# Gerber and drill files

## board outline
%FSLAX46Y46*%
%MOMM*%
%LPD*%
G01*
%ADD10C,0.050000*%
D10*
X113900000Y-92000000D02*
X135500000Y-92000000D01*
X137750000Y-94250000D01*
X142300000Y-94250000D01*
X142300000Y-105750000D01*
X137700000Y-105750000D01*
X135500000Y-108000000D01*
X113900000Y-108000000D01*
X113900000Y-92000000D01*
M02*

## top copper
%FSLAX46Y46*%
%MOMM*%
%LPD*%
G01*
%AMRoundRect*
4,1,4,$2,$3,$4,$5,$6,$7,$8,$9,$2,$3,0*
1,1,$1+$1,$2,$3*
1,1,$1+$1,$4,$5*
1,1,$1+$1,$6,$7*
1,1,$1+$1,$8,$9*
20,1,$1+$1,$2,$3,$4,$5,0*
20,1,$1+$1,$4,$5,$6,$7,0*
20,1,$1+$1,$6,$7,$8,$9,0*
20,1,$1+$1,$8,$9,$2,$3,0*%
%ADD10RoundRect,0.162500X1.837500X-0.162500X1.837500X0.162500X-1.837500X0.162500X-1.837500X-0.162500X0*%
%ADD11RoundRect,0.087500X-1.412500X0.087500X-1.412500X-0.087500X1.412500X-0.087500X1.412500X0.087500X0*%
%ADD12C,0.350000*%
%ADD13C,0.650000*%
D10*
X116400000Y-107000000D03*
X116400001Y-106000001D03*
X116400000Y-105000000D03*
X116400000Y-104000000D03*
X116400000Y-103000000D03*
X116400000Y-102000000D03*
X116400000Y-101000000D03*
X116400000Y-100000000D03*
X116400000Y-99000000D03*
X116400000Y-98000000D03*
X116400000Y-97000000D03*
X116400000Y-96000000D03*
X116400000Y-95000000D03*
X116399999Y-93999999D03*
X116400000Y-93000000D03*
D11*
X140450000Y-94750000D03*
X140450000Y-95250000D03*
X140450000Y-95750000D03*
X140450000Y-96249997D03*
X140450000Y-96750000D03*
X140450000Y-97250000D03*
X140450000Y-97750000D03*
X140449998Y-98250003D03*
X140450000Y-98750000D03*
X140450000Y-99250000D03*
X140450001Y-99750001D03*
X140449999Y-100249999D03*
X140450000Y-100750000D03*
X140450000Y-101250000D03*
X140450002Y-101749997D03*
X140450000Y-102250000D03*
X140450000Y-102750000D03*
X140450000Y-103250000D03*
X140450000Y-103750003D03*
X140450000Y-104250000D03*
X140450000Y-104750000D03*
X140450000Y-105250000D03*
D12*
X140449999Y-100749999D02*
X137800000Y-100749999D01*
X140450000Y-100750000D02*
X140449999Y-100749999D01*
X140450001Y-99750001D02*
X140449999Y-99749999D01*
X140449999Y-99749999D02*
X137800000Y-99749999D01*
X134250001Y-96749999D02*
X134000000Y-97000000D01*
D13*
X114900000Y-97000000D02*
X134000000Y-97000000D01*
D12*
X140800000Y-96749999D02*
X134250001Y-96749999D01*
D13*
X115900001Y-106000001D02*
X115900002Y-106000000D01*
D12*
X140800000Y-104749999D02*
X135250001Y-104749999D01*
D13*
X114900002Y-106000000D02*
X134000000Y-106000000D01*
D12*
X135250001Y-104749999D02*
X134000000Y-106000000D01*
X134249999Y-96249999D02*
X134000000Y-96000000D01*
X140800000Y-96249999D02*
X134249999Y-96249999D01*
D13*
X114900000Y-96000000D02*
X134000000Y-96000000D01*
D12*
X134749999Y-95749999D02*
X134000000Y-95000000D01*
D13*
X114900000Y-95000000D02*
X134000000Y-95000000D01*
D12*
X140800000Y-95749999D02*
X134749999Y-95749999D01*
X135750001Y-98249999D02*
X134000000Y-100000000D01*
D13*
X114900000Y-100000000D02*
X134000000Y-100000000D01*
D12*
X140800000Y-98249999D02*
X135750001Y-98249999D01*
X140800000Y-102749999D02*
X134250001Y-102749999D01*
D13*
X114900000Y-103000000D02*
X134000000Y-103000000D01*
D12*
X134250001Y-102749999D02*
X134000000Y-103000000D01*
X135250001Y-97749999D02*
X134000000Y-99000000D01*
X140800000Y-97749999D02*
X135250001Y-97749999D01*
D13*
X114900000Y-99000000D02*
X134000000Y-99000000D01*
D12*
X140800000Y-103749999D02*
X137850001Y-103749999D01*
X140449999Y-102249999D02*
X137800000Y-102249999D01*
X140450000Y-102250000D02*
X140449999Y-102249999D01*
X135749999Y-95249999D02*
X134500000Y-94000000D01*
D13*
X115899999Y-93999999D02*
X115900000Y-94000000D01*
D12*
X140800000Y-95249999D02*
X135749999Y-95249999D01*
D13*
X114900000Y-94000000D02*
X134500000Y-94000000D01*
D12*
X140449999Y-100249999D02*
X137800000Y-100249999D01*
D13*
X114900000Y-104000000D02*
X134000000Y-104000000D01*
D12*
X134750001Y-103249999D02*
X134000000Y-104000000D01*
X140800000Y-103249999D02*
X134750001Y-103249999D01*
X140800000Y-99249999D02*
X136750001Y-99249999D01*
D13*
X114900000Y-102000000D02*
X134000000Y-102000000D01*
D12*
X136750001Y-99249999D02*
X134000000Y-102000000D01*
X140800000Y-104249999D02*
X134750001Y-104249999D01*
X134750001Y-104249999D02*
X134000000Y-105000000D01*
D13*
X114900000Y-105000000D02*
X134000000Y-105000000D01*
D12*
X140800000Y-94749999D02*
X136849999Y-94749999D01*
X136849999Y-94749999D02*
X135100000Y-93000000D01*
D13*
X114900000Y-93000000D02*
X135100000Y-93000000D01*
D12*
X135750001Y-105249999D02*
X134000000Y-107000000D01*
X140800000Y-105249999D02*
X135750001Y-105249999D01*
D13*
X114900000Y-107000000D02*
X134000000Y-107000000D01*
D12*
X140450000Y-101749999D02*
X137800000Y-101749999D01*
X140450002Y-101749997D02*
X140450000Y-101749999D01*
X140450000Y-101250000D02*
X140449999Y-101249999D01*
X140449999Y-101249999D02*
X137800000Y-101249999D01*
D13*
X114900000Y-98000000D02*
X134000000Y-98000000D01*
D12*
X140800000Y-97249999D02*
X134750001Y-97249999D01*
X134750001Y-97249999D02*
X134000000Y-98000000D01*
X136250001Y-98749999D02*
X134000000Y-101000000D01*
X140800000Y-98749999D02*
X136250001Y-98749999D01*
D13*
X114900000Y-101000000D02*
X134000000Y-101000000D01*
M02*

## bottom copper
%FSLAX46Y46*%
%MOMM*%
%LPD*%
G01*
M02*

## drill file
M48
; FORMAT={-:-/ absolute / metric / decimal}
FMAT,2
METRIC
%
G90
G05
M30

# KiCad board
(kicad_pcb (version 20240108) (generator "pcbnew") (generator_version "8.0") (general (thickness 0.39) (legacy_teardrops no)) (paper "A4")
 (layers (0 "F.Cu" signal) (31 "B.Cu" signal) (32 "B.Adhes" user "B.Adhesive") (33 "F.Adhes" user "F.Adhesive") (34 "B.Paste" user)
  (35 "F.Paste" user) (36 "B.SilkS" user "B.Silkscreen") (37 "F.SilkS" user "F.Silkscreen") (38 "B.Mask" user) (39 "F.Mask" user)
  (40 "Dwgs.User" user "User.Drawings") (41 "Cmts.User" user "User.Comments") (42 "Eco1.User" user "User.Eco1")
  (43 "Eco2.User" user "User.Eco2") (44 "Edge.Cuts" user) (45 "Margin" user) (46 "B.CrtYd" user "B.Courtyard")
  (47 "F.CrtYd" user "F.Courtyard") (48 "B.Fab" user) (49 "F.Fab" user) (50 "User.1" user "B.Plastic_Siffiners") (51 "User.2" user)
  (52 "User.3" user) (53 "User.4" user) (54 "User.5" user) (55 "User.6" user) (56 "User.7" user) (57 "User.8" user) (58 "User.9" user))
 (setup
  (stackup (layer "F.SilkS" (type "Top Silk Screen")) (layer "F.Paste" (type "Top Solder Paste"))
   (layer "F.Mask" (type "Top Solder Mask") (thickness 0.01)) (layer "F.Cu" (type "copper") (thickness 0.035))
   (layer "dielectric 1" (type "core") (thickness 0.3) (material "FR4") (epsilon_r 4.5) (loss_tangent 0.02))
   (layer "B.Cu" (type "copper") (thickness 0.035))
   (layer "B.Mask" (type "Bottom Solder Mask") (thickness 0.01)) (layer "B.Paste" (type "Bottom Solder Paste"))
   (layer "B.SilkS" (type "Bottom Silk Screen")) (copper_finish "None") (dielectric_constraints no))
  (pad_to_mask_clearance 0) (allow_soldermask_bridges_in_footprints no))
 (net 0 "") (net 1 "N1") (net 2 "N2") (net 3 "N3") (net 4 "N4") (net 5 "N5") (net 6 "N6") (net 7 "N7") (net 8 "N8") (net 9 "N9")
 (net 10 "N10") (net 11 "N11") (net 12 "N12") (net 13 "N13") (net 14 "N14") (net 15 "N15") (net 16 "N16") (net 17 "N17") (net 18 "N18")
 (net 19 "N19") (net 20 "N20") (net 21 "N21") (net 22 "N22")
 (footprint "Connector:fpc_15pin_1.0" (layer "F.Cu") (at 116.4 100 90)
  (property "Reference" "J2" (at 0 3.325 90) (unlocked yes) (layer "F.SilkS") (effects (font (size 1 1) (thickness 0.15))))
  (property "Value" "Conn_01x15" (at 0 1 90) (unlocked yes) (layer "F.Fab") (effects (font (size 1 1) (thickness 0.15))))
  (pad "1" smd roundrect (at -7 0 90) (size 0.65 4) (layers "F.Cu" "F.Paste" "F.Mask") (roundrect_rratio 0.25) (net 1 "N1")
   (thermal_bridge_angle 45))
  (pad "2" smd roundrect (at -6.000001 0.000001 90) (size 0.65 4) (layers "F.Cu" "F.Paste" "F.Mask") (roundrect_rratio 0.25) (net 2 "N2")
   (thermal_bridge_angle 45))
  (pad "3" smd roundrect (at -5 0 90) (size 0.65 4) (layers "F.Cu" "F.Paste" "F.Mask") (roundrect_rratio 0.25) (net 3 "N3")
   (thermal_bridge_angle 45))
  (pad "4" smd roundrect (at -4 0 90) (size 0.65 4) (layers "F.Cu" "F.Paste" "F.Mask") (roundrect_rratio 0.25) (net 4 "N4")
   (thermal_bridge_angle 45))
  (pad "5" smd roundrect (at -3 0 90) (size 0.65 4) (layers "F.Cu" "F.Paste" "F.Mask") (roundrect_rratio 0.25) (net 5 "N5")
   (thermal_bridge_angle 45))
  (pad "6" smd roundrect (at -2 0 90) (size 0.65 4) (layers "F.Cu" "F.Paste" "F.Mask") (roundrect_rratio 0.25) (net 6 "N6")
   (thermal_bridge_angle 45))
  (pad "7" smd roundrect (at -1 0 90) (size 0.65 4) (layers "F.Cu" "F.Paste" "F.Mask") (roundrect_rratio 0.25) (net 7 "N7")
   (thermal_bridge_angle 45))
  (pad "8" smd roundrect (at 0 0 90) (size 0.65 4) (layers "F.Cu" "F.Paste" "F.Mask") (roundrect_rratio 0.25) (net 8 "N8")
   (thermal_bridge_angle 45))
  (pad "9" smd roundrect (at 1 0 90) (size 0.65 4) (layers "F.Cu" "F.Paste" "F.Mask") (roundrect_rratio 0.25) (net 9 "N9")
   (thermal_bridge_angle 45))
  (pad "10" smd roundrect (at 2 0 90) (size 0.65 4) (layers "F.Cu" "F.Paste" "F.Mask") (roundrect_rratio 0.25) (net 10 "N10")
   (thermal_bridge_angle 45))
  (pad "11" smd roundrect (at 3 0 90) (size 0.65 4) (layers "F.Cu" "F.Paste" "F.Mask") (roundrect_rratio 0.25) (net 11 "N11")
   (thermal_bridge_angle 45))
  (pad "12" smd roundrect (at 4 0 90) (size 0.65 4) (layers "F.Cu" "F.Paste" "F.Mask") (roundrect_rratio 0.25) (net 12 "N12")
   (thermal_bridge_angle 45))
  (pad "13" smd roundrect (at 5 0 90) (size 0.65 4) (layers "F.Cu" "F.Paste" "F.Mask") (roundrect_rratio 0.25) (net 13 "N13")
   (thermal_bridge_angle 45))
  (pad "14" smd roundrect (at 6.000001 -0.000001 90) (size 0.65 4) (layers "F.Cu" "F.Paste" "F.Mask") (roundrect_rratio 0.25) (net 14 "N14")
   (thermal_bridge_angle 45))
  (pad "15" smd roundrect (at 7 0 90) (size 0.65 4) (layers "F.Cu" "F.Paste" "F.Mask") (roundrect_rratio 0.25) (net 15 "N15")
   (thermal_bridge_angle 45)))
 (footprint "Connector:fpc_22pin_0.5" (layer "F.Cu") (at 140.45 100 -90)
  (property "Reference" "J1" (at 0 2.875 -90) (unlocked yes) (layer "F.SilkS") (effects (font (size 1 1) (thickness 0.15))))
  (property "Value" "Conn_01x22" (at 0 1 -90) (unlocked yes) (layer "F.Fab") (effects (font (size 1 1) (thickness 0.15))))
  (pad "1" smd roundrect (at -5.25 0 270) (size 0.35 3) (layers "F.Cu" "F.Paste" "F.Mask") (roundrect_rratio 0.25) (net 15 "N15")
   (thermal_bridge_angle 45))
  (pad "2" smd roundrect (at -4.75 0 270) (size 0.35 3) (layers "F.Cu" "F.Paste" "F.Mask") (roundrect_rratio 0.25) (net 14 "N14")
   (thermal_bridge_angle 45))
  (pad "3" smd roundrect (at -4.25 0 270) (size 0.35 3) (layers "F.Cu" "F.Paste" "F.Mask") (roundrect_rratio 0.25) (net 13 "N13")
   (thermal_bridge_angle 45))
  (pad "4" smd roundrect (at -3.750003 0 270) (size 0.35 3) (layers "F.Cu" "F.Paste" "F.Mask") (roundrect_rratio 0.25) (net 12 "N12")
   (thermal_bridge_angle 45))
  (pad "5" smd roundrect (at -3.25 0 270) (size 0.35 3) (layers "F.Cu" "F.Paste" "F.Mask") (roundrect_rratio 0.25) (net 11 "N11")
   (thermal_bridge_angle 45))
  (pad "6" smd roundrect (at -2.75 0 270) (size 0.35 3) (layers "F.Cu" "F.Paste" "F.Mask") (roundrect_rratio 0.25) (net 10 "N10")
   (thermal_bridge_angle 45))
  (pad "7" smd roundrect (at -2.25 0 270) (size 0.35 3) (layers "F.Cu" "F.Paste" "F.Mask") (roundrect_rratio 0.25) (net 9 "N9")
   (thermal_bridge_angle 45))
  (pad "8" smd roundrect (at -1.749997 0.000002 270) (size 0.35 3) (layers "F.Cu" "F.Paste" "F.Mask") (roundrect_rratio 0.25) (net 8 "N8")
   (thermal_bridge_angle 45))
  (pad "9" smd roundrect (at -1.25 0 270) (size 0.35 3) (layers "F.Cu" "F.Paste" "F.Mask") (roundrect_rratio 0.25) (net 7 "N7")
   (thermal_bridge_angle 45))
  (pad "10" smd roundrect (at -0.75 0 270) (size 0.35 3) (layers "F.Cu" "F.Paste" "F.Mask") (roundrect_rratio 0.25) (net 6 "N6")
   (thermal_bridge_angle 45))
  (pad "11" smd roundrect (at -0.249999 -0.000001 270) (size 0.35 3) (layers "F.Cu" "F.Paste" "F.Mask") (roundrect_rratio 0.25)
   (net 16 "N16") (thermal_bridge_angle 45))
  (pad "12" smd roundrect (at 0.249999 0.000001 270) (size 0.35 3) (layers "F.Cu" "F.Paste" "F.Mask") (roundrect_rratio 0.25) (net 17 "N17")
   (thermal_bridge_angle 45))
  (pad "13" smd roundrect (at 0.75 0 270) (size 0.35 3) (layers "F.Cu" "F.Paste" "F.Mask") (roundrect_rratio 0.25) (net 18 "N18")
   (thermal_bridge_angle 45))
  (pad "14" smd roundrect (at 1.25 0 270) (size 0.35 3) (layers "F.Cu" "F.Paste" "F.Mask") (roundrect_rratio 0.25) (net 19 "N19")
   (thermal_bridge_angle 45))
  (pad "15" smd roundrect (at 1.749997 -0.000002 270) (size 0.35 3) (layers "F.Cu" "F.Paste" "F.Mask") (roundrect_rratio 0.25)
   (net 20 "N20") (thermal_bridge_angle 45))
  (pad "16" smd roundrect (at 2.25 0 270) (size 0.35 3) (layers "F.Cu" "F.Paste" "F.Mask") (roundrect_rratio 0.25) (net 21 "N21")
   (thermal_bridge_angle 45))
  (pad "17" smd roundrect (at 2.75 0 270) (size 0.35 3) (layers "F.Cu" "F.Paste" "F.Mask") (roundrect_rratio 0.25) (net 5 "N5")
   (thermal_bridge_angle 45))
  (pad "18" smd roundrect (at 3.25 0 270) (size 0.35 3) (layers "F.Cu" "F.Paste" "F.Mask") (roundrect_rratio 0.25) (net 4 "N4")
   (thermal_bridge_angle 45))
  (pad "19" smd roundrect (at 3.750003 0 270) (size 0.35 3) (layers "F.Cu" "F.Paste" "F.Mask") (roundrect_rratio 0.25) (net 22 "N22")
   (thermal_bridge_angle 45))
  (pad "20" smd roundrect (at 4.25 0 270) (size 0.35 3) (layers "F.Cu" "F.Paste" "F.Mask") (roundrect_rratio 0.25) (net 3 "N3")
   (thermal_bridge_angle 45))
  (pad "21" smd roundrect (at 4.75 0 270) (size 0.35 3) (layers "F.Cu" "F.Paste" "F.Mask") (roundrect_rratio 0.25) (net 2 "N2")
   (thermal_bridge_angle 45))
  (pad "22" smd roundrect (at 5.25 0 270) (size 0.35 3) (layers "F.Cu" "F.Paste" "F.Mask") (roundrect_rratio 0.25) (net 1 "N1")
   (thermal_bridge_angle 45)))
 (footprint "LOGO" (layer "F.Cu") (at 123.25 100)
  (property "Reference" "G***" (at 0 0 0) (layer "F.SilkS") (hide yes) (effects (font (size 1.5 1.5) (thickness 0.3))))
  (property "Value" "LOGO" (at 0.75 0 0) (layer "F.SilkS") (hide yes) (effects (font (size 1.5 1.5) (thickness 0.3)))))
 (gr_poly
  (pts (xy 113.9 92) (xy 135.5 92) (xy 137.75 94.25) (xy 142.3 94.25) (xy 142.3 105.75) (xy 137.7 105.75) (xy 135.5 108) (xy 113.9 108))
  (stroke (width 0.05) (type solid)) (fill none) (layer "Edge.Cuts"))
 (segment (start 140.449999 100.749999) (end 137.8 100.749999) (width 0.35) (layer "F.Cu") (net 18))
 (segment (start 140.45 100.75) (end 140.449999 100.749999) (width 0.35) (layer "F.Cu") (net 18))
 (segment (start 140.450001 99.750001) (end 140.449999 99.749999) (width 0.35) (layer "F.Cu") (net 16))
 (segment (start 140.449999 99.749999) (end 137.8 99.749999) (width 0.35) (layer "F.Cu") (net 16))
 (segment (start 134.250001 96.749999) (end 134 97) (width 0.35) (layer "F.Cu") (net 11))
 (segment (start 114.9 97) (end 134 97) (width 0.65) (layer "F.Cu") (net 11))
 (segment (start 140.8 96.749999) (end 134.250001 96.749999) (width 0.35) (layer "F.Cu") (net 11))
 (segment (start 115.900001 106.000001) (end 115.900002 106) (width 0.65) (layer "F.Cu") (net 2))
 (segment (start 140.8 104.749999) (end 135.250001 104.749999) (width 0.35) (layer "F.Cu") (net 2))
 (segment (start 114.900002 106) (end 134 106) (width 0.65) (layer "F.Cu") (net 2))
 (segment (start 135.250001 104.749999) (end 134 106) (width 0.35) (layer "F.Cu") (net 2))
 (segment (start 134.249999 96.249999) (end 134 96) (width 0.35) (layer "F.Cu") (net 12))
 (segment (start 140.8 96.249999) (end 134.249999 96.249999) (width 0.35) (layer "F.Cu") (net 12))
 (segment (start 114.9 96) (end 134 96) (width 0.65) (layer "F.Cu") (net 12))
 (segment (start 134.749999 95.749999) (end 134 95) (width 0.35) (layer "F.Cu") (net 13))
 (segment (start 114.9 95) (end 134 95) (width 0.65) (layer "F.Cu") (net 13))
 (segment (start 140.8 95.749999) (end 134.749999 95.749999) (width 0.35) (layer "F.Cu") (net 13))
 (segment (start 135.750001 98.249999) (end 134 100) (width 0.35) (layer "F.Cu") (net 8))
 (segment (start 114.9 100) (end 134 100) (width 0.65) (layer "F.Cu") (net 8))
 (segment (start 140.8 98.249999) (end 135.750001 98.249999) (width 0.35) (layer "F.Cu") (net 8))
 (segment (start 140.8 102.749999) (end 134.250001 102.749999) (width 0.35) (layer "F.Cu") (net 5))
 (segment (start 114.9 103) (end 134 103) (width 0.65) (layer "F.Cu") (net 5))
 (segment (start 134.250001 102.749999) (end 134 103) (width 0.35) (layer "F.Cu") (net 5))
 (segment (start 135.250001 97.749999) (end 134 99) (width 0.35) (layer "F.Cu") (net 9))
 (segment (start 140.8 97.749999) (end 135.250001 97.749999) (width 0.35) (layer "F.Cu") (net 9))
 (segment (start 114.9 99) (end 134 99) (width 0.65) (layer "F.Cu") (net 9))
 (segment (start 140.8 103.749999) (end 137.850001 103.749999) (width 0.35) (layer "F.Cu") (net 22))
 (segment (start 140.449999 102.249999) (end 137.8 102.249999) (width 0.35) (layer "F.Cu") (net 21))
 (segment (start 140.45 102.25) (end 140.449999 102.249999) (width 0.35) (layer "F.Cu") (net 21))
 (segment (start 135.749999 95.249999) (end 134.5 94) (width 0.35) (layer "F.Cu") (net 14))
 (segment (start 115.899999 93.999999) (end 115.9 94) (width 0.65) (layer "F.Cu") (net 14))
 (segment (start 140.8 95.249999) (end 135.749999 95.249999) (width 0.35) (layer "F.Cu") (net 14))
 (segment (start 114.9 94) (end 134.5 94) (width 0.65) (layer "F.Cu") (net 14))
 (segment (start 140.449999 100.249999) (end 137.8 100.249999) (width 0.35) (layer "F.Cu") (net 17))
 (segment (start 114.9 104) (end 134 104) (width 0.65) (layer "F.Cu") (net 4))
 (segment (start 134.750001 103.249999) (end 134 104) (width 0.35) (layer "F.Cu") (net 4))
 (segment (start 140.8 103.249999) (end 134.750001 103.249999) (width 0.35) (layer "F.Cu") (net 4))
 (segment (start 140.8 99.249999) (end 136.750001 99.249999) (width 0.35) (layer "F.Cu") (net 6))
 (segment (start 114.9 102) (end 134 102) (width 0.65) (layer "F.Cu") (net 6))
 (segment (start 136.750001 99.249999) (end 134 102) (width 0.35) (layer "F.Cu") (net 6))
 (segment (start 140.8 104.249999) (end 134.750001 104.249999) (width 0.35) (layer "F.Cu") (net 3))
 (segment (start 134.750001 104.249999) (end 134 105) (width 0.35) (layer "F.Cu") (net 3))
 (segment (start 114.9 105) (end 134 105) (width 0.65) (layer "F.Cu") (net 3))
 (segment (start 140.8 94.749999) (end 136.849999 94.749999) (width 0.35) (layer "F.Cu") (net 15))
 (segment (start 136.849999 94.749999) (end 135.1 93) (width 0.35) (layer "F.Cu") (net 15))
 (segment (start 114.9 93) (end 135.1 93) (width 0.65) (layer "F.Cu") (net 15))
 (segment (start 135.750001 105.249999) (end 134 107) (width 0.35) (layer "F.Cu") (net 1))
 (segment (start 140.8 105.249999) (end 135.750001 105.249999) (width 0.35) (layer "F.Cu") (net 1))
 (segment (start 114.9 107) (end 134 107) (width 0.65) (layer "F.Cu") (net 1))
 (segment (start 140.45 101.749999) (end 137.8 101.749999) (width 0.35) (layer "F.Cu") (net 20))
 (segment (start 140.450002 101.749997) (end 140.45 101.749999) (width 0.35) (layer "F.Cu") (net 20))
 (segment (start 140.45 101.25) (end 140.449999 101.249999) (width 0.35) (layer "F.Cu") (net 19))
 (segment (start 140.449999 101.249999) (end 137.8 101.249999) (width 0.35) (layer "F.Cu") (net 19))
 (segment (start 114.9 98) (end 134 98) (width 0.65) (layer "F.Cu") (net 10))
 (segment (start 140.8 97.249999) (end 134.750001 97.249999) (width 0.35) (layer "F.Cu") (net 10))
 (segment (start 134.750001 97.249999) (end 134 98) (width 0.35) (layer "F.Cu") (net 10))
 (segment (start 136.250001 98.749999) (end 134 101) (width 0.35) (layer "F.Cu") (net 7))
 (segment (start 140.8 98.749999) (end 136.250001 98.749999) (width 0.35) (layer "F.Cu") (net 7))
 (segment (start 114.9 101) (end 134 101) (width 0.65) (layer "F.Cu") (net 7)))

